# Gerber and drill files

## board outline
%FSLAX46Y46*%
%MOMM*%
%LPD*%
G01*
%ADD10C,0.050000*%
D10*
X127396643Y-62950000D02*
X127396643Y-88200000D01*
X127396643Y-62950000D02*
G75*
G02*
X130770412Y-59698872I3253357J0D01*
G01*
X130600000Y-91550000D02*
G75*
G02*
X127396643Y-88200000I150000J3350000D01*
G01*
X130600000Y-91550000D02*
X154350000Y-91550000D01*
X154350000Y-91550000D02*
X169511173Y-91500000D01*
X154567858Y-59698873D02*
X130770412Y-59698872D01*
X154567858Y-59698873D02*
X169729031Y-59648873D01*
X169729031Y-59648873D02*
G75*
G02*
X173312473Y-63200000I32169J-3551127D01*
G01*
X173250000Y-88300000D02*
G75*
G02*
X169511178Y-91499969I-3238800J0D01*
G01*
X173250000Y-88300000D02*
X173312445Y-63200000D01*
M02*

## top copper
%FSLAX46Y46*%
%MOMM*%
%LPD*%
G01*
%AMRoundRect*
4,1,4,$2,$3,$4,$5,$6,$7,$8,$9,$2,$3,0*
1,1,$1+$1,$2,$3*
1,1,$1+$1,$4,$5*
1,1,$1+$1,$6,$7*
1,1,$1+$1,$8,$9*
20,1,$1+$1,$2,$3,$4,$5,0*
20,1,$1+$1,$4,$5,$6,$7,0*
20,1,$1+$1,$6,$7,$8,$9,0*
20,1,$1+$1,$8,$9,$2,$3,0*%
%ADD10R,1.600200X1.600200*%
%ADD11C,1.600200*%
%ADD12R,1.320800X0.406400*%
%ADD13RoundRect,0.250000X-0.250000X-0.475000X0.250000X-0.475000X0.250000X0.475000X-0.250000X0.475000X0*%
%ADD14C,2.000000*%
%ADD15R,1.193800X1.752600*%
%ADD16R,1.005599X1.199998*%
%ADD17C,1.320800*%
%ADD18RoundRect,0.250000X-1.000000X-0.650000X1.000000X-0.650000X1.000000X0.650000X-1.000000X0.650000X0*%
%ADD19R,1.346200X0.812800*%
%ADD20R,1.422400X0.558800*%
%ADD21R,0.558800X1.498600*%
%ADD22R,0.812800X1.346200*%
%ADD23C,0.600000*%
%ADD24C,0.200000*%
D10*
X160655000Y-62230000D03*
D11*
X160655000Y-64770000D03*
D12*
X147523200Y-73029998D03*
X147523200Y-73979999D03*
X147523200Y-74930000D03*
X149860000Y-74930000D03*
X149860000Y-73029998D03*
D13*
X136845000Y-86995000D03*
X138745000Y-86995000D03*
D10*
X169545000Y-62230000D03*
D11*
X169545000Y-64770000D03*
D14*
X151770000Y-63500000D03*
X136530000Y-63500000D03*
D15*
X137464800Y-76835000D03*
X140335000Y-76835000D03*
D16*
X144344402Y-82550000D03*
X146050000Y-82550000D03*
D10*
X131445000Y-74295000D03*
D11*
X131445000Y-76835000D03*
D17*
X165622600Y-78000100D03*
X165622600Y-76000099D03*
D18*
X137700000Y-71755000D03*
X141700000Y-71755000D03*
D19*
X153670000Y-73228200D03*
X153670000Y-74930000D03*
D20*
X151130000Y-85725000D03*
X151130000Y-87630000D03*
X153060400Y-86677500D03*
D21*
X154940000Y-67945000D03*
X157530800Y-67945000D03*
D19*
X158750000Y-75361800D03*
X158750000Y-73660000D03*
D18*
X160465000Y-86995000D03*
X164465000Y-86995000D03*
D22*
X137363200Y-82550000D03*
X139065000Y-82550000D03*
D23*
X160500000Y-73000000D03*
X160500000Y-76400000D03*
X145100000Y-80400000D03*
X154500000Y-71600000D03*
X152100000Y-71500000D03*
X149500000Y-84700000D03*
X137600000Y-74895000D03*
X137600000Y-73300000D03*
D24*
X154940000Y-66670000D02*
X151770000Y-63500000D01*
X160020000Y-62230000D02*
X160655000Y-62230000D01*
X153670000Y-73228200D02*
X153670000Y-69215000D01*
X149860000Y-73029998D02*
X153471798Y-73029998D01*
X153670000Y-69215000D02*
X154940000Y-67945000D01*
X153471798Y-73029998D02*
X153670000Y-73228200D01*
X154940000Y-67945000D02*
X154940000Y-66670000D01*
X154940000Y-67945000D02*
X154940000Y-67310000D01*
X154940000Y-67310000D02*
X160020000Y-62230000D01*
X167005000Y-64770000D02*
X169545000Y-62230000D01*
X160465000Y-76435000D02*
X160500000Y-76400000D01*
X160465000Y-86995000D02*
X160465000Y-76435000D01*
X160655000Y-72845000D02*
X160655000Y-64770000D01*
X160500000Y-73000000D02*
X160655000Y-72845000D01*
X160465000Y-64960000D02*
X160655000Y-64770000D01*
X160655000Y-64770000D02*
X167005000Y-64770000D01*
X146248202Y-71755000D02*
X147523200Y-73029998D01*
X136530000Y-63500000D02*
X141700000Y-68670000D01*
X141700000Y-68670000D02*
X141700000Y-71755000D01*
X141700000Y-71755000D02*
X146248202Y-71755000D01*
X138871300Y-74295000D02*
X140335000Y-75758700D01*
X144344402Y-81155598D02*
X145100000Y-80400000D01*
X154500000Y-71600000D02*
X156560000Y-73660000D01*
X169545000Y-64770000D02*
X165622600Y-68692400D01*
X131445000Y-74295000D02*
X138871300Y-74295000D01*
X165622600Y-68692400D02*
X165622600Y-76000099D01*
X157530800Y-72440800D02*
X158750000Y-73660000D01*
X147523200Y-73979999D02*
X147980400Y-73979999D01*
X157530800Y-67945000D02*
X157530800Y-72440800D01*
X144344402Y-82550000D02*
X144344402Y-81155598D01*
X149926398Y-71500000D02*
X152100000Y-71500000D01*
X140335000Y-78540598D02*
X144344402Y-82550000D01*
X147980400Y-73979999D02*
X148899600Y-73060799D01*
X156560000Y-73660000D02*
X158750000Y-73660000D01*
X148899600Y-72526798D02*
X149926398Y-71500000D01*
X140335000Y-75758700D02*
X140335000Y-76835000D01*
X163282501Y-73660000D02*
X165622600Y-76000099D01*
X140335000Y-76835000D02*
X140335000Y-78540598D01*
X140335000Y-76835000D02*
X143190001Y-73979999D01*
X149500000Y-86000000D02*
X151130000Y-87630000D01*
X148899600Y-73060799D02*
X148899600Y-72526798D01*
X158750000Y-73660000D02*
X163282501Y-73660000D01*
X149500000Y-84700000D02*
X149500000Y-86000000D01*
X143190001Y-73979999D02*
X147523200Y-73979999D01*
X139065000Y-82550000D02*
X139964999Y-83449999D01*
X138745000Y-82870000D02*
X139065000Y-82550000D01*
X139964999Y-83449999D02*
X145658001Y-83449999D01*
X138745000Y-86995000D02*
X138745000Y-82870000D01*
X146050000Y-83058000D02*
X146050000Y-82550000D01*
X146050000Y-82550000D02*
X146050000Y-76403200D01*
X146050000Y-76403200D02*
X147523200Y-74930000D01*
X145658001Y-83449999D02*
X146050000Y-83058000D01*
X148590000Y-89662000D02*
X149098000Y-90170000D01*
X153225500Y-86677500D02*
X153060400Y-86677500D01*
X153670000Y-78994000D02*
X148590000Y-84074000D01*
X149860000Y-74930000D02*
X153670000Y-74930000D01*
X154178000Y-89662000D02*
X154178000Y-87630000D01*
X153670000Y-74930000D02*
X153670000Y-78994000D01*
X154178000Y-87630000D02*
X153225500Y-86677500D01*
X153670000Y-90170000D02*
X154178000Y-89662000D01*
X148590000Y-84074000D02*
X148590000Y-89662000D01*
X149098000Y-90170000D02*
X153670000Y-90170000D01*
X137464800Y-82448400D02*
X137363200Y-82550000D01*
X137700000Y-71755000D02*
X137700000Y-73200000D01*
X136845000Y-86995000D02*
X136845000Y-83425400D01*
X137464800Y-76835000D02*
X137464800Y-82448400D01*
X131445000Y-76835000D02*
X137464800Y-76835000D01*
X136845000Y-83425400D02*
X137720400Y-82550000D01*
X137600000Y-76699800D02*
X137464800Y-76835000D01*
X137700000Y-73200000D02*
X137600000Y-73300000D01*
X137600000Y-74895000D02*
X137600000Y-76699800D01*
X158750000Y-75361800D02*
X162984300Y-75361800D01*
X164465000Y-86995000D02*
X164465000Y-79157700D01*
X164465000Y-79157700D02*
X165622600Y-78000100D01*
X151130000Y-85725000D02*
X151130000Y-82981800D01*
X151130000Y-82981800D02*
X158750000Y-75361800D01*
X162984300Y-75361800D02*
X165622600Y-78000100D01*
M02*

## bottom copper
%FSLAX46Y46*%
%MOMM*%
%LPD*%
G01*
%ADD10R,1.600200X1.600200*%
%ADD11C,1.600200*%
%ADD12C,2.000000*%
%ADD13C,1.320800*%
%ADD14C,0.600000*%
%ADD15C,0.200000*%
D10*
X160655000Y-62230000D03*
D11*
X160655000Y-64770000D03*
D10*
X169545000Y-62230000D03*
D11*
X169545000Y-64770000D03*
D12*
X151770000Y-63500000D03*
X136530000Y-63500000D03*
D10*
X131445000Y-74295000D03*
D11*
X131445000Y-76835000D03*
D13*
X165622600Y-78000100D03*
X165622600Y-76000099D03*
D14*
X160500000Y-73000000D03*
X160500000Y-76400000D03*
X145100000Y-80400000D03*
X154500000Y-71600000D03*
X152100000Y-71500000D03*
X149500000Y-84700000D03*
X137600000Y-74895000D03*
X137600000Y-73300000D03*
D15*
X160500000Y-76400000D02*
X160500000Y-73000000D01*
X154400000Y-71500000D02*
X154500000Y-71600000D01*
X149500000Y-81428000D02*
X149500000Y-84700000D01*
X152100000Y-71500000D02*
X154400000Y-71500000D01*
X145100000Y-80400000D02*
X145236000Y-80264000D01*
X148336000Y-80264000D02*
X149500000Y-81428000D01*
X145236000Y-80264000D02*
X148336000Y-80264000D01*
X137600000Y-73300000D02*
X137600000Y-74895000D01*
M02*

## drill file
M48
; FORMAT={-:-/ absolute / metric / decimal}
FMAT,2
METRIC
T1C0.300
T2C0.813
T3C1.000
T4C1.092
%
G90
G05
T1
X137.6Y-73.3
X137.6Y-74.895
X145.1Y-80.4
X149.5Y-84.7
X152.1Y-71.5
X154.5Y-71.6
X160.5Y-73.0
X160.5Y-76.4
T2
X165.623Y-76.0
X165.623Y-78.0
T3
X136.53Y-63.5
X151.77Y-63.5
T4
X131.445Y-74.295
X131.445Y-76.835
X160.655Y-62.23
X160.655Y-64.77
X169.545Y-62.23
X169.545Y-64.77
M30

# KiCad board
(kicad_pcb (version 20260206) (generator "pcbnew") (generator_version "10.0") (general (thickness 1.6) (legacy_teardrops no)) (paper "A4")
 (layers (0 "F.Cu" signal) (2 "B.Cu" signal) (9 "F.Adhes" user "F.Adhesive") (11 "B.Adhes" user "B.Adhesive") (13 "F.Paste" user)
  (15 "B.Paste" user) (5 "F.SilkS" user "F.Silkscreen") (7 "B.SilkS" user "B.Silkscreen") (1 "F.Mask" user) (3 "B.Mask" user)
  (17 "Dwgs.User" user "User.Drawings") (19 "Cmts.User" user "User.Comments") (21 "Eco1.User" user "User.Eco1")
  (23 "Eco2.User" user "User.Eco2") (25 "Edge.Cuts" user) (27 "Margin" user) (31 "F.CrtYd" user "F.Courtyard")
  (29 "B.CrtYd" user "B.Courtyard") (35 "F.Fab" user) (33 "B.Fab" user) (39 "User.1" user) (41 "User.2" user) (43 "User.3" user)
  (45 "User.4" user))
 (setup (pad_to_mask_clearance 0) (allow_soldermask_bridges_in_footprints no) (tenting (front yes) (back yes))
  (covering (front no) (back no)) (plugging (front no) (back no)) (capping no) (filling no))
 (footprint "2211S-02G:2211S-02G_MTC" (layer "F.Cu") (at 160.655 62.23 90)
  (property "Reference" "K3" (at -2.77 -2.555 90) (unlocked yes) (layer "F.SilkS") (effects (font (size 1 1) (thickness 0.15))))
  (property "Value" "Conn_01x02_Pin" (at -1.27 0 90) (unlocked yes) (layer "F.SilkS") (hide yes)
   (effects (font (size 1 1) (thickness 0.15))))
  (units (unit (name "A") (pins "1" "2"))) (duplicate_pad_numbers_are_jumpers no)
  (pad "1" thru_hole rect (at 0 0 90) (size 1.6002 1.6002) (drill 1.0922) (layers "*.Cu" "*.Mask") (remove_unused_layers no) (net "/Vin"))
  (pad "2" thru_hole circle (at -2.54 0 90) (size 1.6002 1.6002) (drill 1.0922) (layers "*.Cu" "*.Mask") (remove_unused_layers no)
   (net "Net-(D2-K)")))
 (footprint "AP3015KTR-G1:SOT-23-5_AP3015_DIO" (layer "F.Cu") (at 148.6916 73.979999)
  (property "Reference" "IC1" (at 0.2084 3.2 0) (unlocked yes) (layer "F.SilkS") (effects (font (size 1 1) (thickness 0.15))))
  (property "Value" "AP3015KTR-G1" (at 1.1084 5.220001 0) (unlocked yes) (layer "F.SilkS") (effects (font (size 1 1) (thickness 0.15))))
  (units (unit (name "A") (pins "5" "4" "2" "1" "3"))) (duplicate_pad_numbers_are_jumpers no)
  (pad "1" smd rect (at -1.1684 -0.950001) (size 1.3208 0.4064) (layers "F.Cu" "F.Mask" "F.Paste") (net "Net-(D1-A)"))
  (pad "2" smd rect (at -1.1684 0) (size 1.3208 0.4064) (layers "F.Cu" "F.Mask" "F.Paste") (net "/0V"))
  (pad "3" smd rect (at -1.1684 0.950001) (size 1.3208 0.4064) (layers "F.Cu" "F.Mask" "F.Paste") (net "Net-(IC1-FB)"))
  (pad "4" smd rect (at 1.1684 0.950001) (size 1.3208 0.4064) (layers "F.Cu" "F.Mask" "F.Paste") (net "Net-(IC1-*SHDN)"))
  (pad "5" smd rect (at 1.1684 -0.950001) (size 1.3208 0.4064) (layers "F.Cu" "F.Mask" "F.Paste") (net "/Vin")))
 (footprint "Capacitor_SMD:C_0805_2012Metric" (layer "F.Cu") (at 137.795 86.995)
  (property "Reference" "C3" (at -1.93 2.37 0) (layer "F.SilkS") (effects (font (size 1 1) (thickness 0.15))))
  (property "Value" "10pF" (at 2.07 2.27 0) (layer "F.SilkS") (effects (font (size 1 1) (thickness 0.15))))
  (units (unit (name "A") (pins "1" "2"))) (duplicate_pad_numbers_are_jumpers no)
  (pad "1" smd roundrect (at -0.95 0) (size 1 1.45) (layers "F.Cu" "F.Mask" "F.Paste") (roundrect_rratio 0.25) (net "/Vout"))
  (pad "2" smd roundrect (at 0.95 0) (size 1 1.45) (layers "F.Cu" "F.Mask" "F.Paste") (roundrect_rratio 0.25) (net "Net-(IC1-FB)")))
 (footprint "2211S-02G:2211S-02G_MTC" (layer "F.Cu") (at 169.545 62.23 90)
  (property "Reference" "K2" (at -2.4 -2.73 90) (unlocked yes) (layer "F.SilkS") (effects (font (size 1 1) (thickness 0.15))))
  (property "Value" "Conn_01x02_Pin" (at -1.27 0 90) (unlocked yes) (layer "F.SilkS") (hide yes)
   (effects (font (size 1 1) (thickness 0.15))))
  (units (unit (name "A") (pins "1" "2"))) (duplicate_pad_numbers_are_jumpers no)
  (pad "1" thru_hole rect (at 0 0 90) (size 1.6002 1.6002) (drill 1.0922) (layers "*.Cu" "*.Mask") (remove_unused_layers no)
   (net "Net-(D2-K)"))
  (pad "2" thru_hole circle (at -2.54 0 90) (size 1.6002 1.6002) (drill 1.0922) (layers "*.Cu" "*.Mask") (remove_unused_layers no)
   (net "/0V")))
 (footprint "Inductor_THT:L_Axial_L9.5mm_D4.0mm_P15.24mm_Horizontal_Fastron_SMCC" (layer "F.Cu") (at 151.77 63.5 180)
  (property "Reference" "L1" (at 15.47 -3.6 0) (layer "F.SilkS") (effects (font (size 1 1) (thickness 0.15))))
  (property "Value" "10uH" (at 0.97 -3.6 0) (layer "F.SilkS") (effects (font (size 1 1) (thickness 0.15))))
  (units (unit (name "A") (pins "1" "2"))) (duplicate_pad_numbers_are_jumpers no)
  (pad "1" thru_hole circle (at 0 0 180) (size 2 2) (drill 1) (layers "*.Cu" "*.Mask") (remove_unused_layers no) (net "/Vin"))
  (pad "2" thru_hole circle (at 15.24 0 180) (size 2 2) (drill 1) (layers "*.Cu" "*.Mask") (remove_unused_layers no) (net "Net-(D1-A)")))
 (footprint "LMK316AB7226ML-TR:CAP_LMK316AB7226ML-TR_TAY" (layer "F.Cu") (at 138.8999 76.835)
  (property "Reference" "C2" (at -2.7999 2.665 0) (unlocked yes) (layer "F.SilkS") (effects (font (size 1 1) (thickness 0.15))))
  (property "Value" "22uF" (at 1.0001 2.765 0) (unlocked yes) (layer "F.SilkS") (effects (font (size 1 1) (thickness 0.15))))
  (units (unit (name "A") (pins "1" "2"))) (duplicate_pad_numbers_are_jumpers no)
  (pad "1" smd rect (at -1.4351 0) (size 1.1938 1.7526) (layers "F.Cu" "F.Mask" "F.Paste") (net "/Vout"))
  (pad "2" smd rect (at 1.4351 0) (size 1.1938 1.7526) (layers "F.Cu" "F.Mask" "F.Paste") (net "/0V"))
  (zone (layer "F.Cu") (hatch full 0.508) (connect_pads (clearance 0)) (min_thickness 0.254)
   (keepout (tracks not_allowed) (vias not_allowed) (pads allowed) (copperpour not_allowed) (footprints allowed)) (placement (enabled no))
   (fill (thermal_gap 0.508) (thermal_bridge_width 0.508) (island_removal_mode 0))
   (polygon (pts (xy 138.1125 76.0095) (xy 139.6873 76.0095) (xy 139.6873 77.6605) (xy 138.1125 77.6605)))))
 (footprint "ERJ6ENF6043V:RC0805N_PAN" (layer "F.Cu") (at 145.197201 82.55)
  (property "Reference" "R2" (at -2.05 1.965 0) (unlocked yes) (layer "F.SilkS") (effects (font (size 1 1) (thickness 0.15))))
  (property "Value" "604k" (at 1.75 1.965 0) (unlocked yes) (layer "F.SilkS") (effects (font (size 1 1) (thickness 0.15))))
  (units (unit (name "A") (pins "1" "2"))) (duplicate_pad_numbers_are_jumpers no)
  (pad "1" smd rect (at -0.852799 0) (size 1.005599 1.199998) (layers "F.Cu" "F.Mask" "F.Paste") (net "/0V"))
  (pad "2" smd rect (at 0.852799 0) (size 1.005599 1.199998) (layers "F.Cu" "F.Mask" "F.Paste") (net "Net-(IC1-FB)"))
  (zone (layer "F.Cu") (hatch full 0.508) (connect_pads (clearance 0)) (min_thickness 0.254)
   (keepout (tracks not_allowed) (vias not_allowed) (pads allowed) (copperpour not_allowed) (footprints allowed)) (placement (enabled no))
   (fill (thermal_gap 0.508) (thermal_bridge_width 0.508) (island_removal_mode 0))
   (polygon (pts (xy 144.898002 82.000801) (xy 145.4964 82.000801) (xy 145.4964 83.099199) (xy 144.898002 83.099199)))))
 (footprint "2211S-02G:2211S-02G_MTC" (layer "F.Cu") (at 131.445 74.295 90)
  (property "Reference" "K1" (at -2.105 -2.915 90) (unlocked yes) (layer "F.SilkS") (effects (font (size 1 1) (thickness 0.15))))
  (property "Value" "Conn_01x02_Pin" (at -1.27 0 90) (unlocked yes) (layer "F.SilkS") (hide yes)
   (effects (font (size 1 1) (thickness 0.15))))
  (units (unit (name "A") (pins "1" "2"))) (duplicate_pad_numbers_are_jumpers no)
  (pad "1" thru_hole rect (at 0 0 90) (size 1.6002 1.6002) (drill 1.0922) (layers "*.Cu" "*.Mask") (remove_unused_layers no) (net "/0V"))
  (pad "2" thru_hole circle (at -2.54 0 90) (size 1.6002 1.6002) (drill 1.0922) (layers "*.Cu" "*.Mask") (remove_unused_layers no)
   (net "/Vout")))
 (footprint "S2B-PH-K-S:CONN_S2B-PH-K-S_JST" (layer "F.Cu") (at 165.6226 78.0001 90)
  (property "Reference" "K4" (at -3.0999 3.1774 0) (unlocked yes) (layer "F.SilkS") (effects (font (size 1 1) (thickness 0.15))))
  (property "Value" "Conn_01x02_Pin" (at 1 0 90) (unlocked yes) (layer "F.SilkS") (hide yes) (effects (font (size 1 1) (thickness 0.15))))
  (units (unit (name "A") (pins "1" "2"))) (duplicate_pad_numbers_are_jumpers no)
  (pad "1" thru_hole circle (at 0 0 90) (size 1.3208 1.3208) (drill 0.8128) (layers "*.Cu" "*.Mask") (remove_unused_layers no) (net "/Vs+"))
  (pad "2" thru_hole circle (at 2.000001 0 90) (size 1.3208 1.3208) (drill 0.8128) (layers "*.Cu" "*.Mask") (remove_unused_layers no)
   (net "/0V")))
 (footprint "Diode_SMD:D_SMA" (layer "F.Cu") (at 139.7 71.755)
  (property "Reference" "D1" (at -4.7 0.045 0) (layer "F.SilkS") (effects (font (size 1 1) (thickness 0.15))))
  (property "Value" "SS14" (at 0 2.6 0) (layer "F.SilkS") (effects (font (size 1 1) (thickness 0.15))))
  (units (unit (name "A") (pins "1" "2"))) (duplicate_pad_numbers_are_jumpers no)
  (pad "1" smd roundrect (at -2 0) (size 2.5 1.8) (layers "F.Cu" "F.Mask" "F.Paste") (roundrect_rratio 0.1388888889) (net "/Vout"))
  (pad "2" smd roundrect (at 2 0) (size 2.5 1.8) (layers "F.Cu" "F.Mask" "F.Paste") (roundrect_rratio 0.1388888889) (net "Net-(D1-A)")))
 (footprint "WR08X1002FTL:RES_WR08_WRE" (layer "F.Cu") (at 153.67 74.0791 -90)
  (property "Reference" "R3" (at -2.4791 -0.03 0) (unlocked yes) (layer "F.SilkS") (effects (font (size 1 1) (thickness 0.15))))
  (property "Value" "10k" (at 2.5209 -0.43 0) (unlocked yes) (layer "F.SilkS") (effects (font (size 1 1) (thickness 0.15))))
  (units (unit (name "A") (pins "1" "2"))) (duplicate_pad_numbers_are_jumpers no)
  (pad "1" smd rect (at -0.8509 0 270) (size 0.8128 1.3462) (layers "F.Cu" "F.Mask" "F.Paste") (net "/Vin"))
  (pad "2" smd rect (at 0.8509 0 270) (size 0.8128 1.3462) (layers "F.Cu" "F.Mask" "F.Paste") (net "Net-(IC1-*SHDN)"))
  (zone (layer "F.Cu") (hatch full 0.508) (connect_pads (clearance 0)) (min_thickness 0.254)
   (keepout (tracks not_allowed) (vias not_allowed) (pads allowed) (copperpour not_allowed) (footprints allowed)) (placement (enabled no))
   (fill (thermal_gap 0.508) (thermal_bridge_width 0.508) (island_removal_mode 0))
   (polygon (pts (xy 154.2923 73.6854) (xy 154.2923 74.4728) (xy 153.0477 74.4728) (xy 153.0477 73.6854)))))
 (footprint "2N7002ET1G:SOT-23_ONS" (layer "F.Cu") (at 152.0952 86.6775 -90)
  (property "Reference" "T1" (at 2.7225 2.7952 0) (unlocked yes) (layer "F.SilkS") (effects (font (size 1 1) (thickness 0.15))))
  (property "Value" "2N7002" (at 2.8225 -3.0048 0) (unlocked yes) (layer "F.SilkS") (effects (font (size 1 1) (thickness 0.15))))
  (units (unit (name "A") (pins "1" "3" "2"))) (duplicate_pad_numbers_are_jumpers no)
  (pad "1" smd rect (at -0.9525 0.9652 270) (size 0.5588 1.4224) (layers "F.Cu" "F.Mask" "F.Paste") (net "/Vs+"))
  (pad "2" smd rect (at 0.9525 0.9652 270) (size 0.5588 1.4224) (layers "F.Cu" "F.Mask" "F.Paste") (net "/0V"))
  (pad "3" smd rect (at 0 -0.9652 270) (size 0.5588 1.4224) (layers "F.Cu" "F.Mask" "F.Paste") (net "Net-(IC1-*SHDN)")))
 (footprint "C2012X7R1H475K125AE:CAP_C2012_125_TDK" (layer "F.Cu") (at 156.2354 67.945)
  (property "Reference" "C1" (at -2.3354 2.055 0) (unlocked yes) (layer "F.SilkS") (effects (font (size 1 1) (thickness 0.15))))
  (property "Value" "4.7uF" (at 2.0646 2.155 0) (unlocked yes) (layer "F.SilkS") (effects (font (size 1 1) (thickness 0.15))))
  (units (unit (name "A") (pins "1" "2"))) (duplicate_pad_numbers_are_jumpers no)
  (pad "1" smd rect (at -1.2954 0) (size 0.5588 1.4986) (layers "F.Cu" "F.Mask" "F.Paste") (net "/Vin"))
  (pad "2" smd rect (at 1.2954 0) (size 0.5588 1.4986) (layers "F.Cu" "F.Mask" "F.Paste") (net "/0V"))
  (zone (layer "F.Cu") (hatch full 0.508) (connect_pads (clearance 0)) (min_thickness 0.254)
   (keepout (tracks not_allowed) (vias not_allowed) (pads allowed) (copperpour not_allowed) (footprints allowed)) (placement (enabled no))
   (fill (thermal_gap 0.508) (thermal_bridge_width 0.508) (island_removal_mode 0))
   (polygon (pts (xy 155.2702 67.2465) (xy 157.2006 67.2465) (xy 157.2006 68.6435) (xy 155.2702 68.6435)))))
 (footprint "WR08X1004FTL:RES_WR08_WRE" (layer "F.Cu") (at 158.75 74.5109 90)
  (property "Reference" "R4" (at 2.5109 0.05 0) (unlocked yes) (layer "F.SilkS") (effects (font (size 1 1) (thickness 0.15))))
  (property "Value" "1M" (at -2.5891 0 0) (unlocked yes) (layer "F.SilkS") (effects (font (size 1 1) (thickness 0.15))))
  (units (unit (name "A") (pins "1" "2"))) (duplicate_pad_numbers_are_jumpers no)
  (pad "1" smd rect (at -0.8509 0 90) (size 0.8128 1.3462) (layers "F.Cu" "F.Mask" "F.Paste") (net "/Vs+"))
  (pad "2" smd rect (at 0.8509 0 90) (size 0.8128 1.3462) (layers "F.Cu" "F.Mask" "F.Paste") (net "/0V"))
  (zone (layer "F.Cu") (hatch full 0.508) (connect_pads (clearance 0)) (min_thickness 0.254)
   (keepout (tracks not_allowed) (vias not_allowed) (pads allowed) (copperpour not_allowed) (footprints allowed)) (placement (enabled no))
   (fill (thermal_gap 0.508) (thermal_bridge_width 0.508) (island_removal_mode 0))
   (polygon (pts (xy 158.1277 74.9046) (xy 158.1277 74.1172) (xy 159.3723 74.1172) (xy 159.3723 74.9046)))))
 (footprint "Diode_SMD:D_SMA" (layer "F.Cu") (at 162.465 86.995)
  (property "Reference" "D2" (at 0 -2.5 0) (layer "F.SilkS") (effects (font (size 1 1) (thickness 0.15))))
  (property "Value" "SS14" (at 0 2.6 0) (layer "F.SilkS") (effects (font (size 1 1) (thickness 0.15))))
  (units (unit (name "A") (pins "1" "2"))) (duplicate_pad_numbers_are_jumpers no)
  (pad "1" smd roundrect (at -2 0) (size 2.5 1.8) (layers "F.Cu" "F.Mask" "F.Paste") (roundrect_rratio 0.1388888889) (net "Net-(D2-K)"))
  (pad "2" smd roundrect (at 2 0) (size 2.5 1.8) (layers "F.Cu" "F.Mask" "F.Paste") (roundrect_rratio 0.1388888889) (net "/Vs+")))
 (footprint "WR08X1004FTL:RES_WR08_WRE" (layer "F.Cu") (at 138.2141 82.55)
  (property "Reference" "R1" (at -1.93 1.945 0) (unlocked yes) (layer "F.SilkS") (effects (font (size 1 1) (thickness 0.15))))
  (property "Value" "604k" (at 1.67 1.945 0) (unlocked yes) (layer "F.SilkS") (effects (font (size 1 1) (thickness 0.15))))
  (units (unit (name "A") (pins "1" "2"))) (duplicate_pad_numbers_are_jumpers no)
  (pad "1" smd rect (at -0.8509 0) (size 0.8128 1.3462) (layers "F.Cu" "F.Mask" "F.Paste") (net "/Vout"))
  (pad "2" smd rect (at 0.8509 0) (size 0.8128 1.3462) (layers "F.Cu" "F.Mask" "F.Paste") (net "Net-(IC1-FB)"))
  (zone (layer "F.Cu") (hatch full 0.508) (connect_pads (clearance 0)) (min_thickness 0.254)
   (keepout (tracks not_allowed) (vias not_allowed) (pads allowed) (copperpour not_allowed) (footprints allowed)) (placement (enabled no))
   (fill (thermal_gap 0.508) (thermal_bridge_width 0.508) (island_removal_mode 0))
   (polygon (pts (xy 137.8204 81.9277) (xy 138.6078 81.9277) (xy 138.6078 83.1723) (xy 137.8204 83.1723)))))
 (gr_line (start 127.396643 62.95) (end 127.396643 88.2) (stroke (width 0.05) (type default)) (layer "Edge.Cuts"))
 (gr_arc (start 127.396643 62.95) (mid 128.392503 60.607344) (end 130.770412 59.698872) (stroke (width 0.05) (type default))
  (layer "Edge.Cuts"))
 (gr_arc (start 130.6 91.55) (mid 128.326366 90.517541) (end 127.396643 88.2) (stroke (width 0.05) (type default)) (layer "Edge.Cuts"))
 (gr_line (start 130.6 91.55) (end 154.35 91.55) (stroke (width 0.05) (type default)) (layer "Edge.Cuts"))
 (gr_line (start 154.35 91.55) (end 169.511173 91.5) (stroke (width 0.05) (type default)) (layer "Edge.Cuts"))
 (gr_line (start 154.567858 59.698873) (end 130.770412 59.698872) (stroke (width 0.05) (type default)) (layer "Edge.Cuts"))
 (gr_line (start 154.567858 59.698873) (end 169.729031 59.648873) (stroke (width 0.05) (type default)) (layer "Edge.Cuts"))
 (gr_arc (start 169.729031 59.648873) (mid 172.260912 60.677533) (end 173.312445 63.2) (stroke (width 0.05) (type default))
  (layer "Edge.Cuts"))
 (gr_arc (start 173.25 88.3) (mid 172.117187 90.760631) (end 169.511173 91.5) (stroke (width 0.05) (type default)) (layer "Edge.Cuts"))
 (gr_line (start 173.25 88.3) (end 173.312445 63.2) (stroke (width 0.05) (type default)) (layer "Edge.Cuts"))
 (segment (start 154.94 66.67) (end 151.77 63.5) (width 0.2) (layer "F.Cu") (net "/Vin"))
 (segment (start 160.02 62.23) (end 160.655 62.23) (width 0.2) (layer "F.Cu") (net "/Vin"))
 (segment (start 153.67 73.2282) (end 153.67 69.215) (width 0.2) (layer "F.Cu") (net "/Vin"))
 (segment (start 149.86 73.029998) (end 153.471798 73.029998) (width 0.2) (layer "F.Cu") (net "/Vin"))
 (segment (start 153.67 69.215) (end 154.94 67.945) (width 0.2) (layer "F.Cu") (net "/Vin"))
 (segment (start 153.471798 73.029998) (end 153.67 73.2282) (width 0.2) (layer "F.Cu") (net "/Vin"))
 (segment (start 154.94 67.945) (end 154.94 66.67) (width 0.2) (layer "F.Cu") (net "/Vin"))
 (segment (start 154.94 67.945) (end 154.94 67.31) (width 0.2) (layer "F.Cu") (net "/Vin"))
 (segment (start 154.94 67.31) (end 160.02 62.23) (width 0.2) (layer "F.Cu") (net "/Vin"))
 (segment (start 167.005 64.77) (end 169.545 62.23) (width 0.2) (layer "F.Cu") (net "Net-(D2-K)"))
 (segment (start 160.465 76.435) (end 160.5 76.4) (width 0.2) (layer "F.Cu") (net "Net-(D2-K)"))
 (segment (start 160.465 86.995) (end 160.465 76.435) (width 0.2) (layer "F.Cu") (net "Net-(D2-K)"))
 (segment (start 160.655 72.845) (end 160.655 64.77) (width 0.2) (layer "F.Cu") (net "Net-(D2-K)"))
 (segment (start 160.5 73) (end 160.655 72.845) (width 0.2) (layer "F.Cu") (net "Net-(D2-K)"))
 (segment (start 160.465 64.96) (end 160.655 64.77) (width 0.2) (layer "F.Cu") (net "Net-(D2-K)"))
 (segment (start 160.655 64.77) (end 167.005 64.77) (width 0.2) (layer "F.Cu") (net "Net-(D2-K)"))
 (via (at 160.5 73) (size 0.6) (drill 0.3) (layers "F.Cu" "B.Cu") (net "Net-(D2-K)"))
 (via (at 160.5 76.4) (size 0.6) (drill 0.3) (layers "F.Cu" "B.Cu") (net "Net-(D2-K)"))
 (segment (start 160.5 76.4) (end 160.5 73) (width 0.2) (layer "B.Cu") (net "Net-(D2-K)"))
 (segment (start 146.248202 71.755) (end 147.5232 73.029998) (width 0.2) (layer "F.Cu") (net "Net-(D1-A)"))
 (segment (start 136.53 63.5) (end 141.7 68.67) (width 0.2) (layer "F.Cu") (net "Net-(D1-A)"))
 (segment (start 141.7 68.67) (end 141.7 71.755) (width 0.2) (layer "F.Cu") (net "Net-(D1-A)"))
 (segment (start 141.7 71.755) (end 146.248202 71.755) (width 0.2) (layer "F.Cu") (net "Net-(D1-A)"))
 (segment (start 138.8713 74.295) (end 140.335 75.7587) (width 0.2) (layer "F.Cu") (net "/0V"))
 (segment (start 144.344402 81.155598) (end 145.1 80.4) (width 0.2) (layer "F.Cu") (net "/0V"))
 (segment (start 154.5 71.6) (end 156.56 73.66) (width 0.2) (layer "F.Cu") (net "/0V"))
 (segment (start 169.545 64.77) (end 165.6226 68.6924) (width 0.2) (layer "F.Cu") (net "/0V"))
 (segment (start 131.445 74.295) (end 138.8713 74.295) (width 0.2) (layer "F.Cu") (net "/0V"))
 (segment (start 165.6226 68.6924) (end 165.6226 76.000099) (width 0.2) (layer "F.Cu") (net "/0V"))
 (segment (start 157.5308 72.4408) (end 158.75 73.66) (width 0.2) (layer "F.Cu") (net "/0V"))
 (segment (start 147.5232 73.979999) (end 147.9804 73.979999) (width 0.2) (layer "F.Cu") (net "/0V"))
 (segment (start 157.5308 67.945) (end 157.5308 72.4408) (width 0.2) (layer "F.Cu") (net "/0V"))
 (segment (start 144.344402 82.55) (end 144.344402 81.155598) (width 0.2) (layer "F.Cu") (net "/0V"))
 (segment (start 149.926398 71.5) (end 152.1 71.5) (width 0.2) (layer "F.Cu") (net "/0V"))
 (segment (start 140.335 78.540598) (end 144.344402 82.55) (width 0.2) (layer "F.Cu") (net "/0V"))
 (segment (start 147.9804 73.979999) (end 148.8996 73.060799) (width 0.2) (layer "F.Cu") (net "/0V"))
 (segment (start 156.56 73.66) (end 158.75 73.66) (width 0.2) (layer "F.Cu") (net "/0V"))
 (segment (start 148.8996 72.526798) (end 149.926398 71.5) (width 0.2) (layer "F.Cu") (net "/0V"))
 (segment (start 140.335 75.7587) (end 140.335 76.835) (width 0.2) (layer "F.Cu") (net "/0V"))
 (segment (start 163.282501 73.66) (end 165.6226 76.000099) (width 0.2) (layer "F.Cu") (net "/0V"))
 (segment (start 140.335 76.835) (end 140.335 78.540598) (width 0.2) (layer "F.Cu") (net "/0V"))
 (segment (start 140.335 76.835) (end 143.190001 73.979999) (width 0.2) (layer "F.Cu") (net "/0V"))
 (segment (start 149.5 86) (end 151.13 87.63) (width 0.2) (layer "F.Cu") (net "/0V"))
 (segment (start 148.8996 73.060799) (end 148.8996 72.526798) (width 0.2) (layer "F.Cu") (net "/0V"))
 (segment (start 158.75 73.66) (end 163.282501 73.66) (width 0.2) (layer "F.Cu") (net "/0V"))
 (segment (start 149.5 84.7) (end 149.5 86) (width 0.2) (layer "F.Cu") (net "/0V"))
 (segment (start 143.190001 73.979999) (end 147.5232 73.979999) (width 0.2) (layer "F.Cu") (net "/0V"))
 (via (at 145.1 80.4) (size 0.6) (drill 0.3) (layers "F.Cu" "B.Cu") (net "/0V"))
 (via (at 154.5 71.6) (size 0.6) (drill 0.3) (layers "F.Cu" "B.Cu") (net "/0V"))
 (via (at 152.1 71.5) (size 0.6) (drill 0.3) (layers "F.Cu" "B.Cu") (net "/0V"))
 (via (at 149.5 84.7) (size 0.6) (drill 0.3) (layers "F.Cu" "B.Cu") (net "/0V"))
 (segment (start 154.4 71.5) (end 154.5 71.6) (width 0.2) (layer "B.Cu") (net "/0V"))
 (segment (start 149.5 81.428) (end 149.5 84.7) (width 0.2) (layer "B.Cu") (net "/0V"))
 (segment (start 152.1 71.5) (end 154.4 71.5) (width 0.2) (layer "B.Cu") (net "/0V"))
 (segment (start 145.1 80.4) (end 145.236 80.264) (width 0.2) (layer "B.Cu") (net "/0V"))
 (segment (start 148.336 80.264) (end 149.5 81.428) (width 0.2) (layer "B.Cu") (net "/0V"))
 (segment (start 145.236 80.264) (end 148.336 80.264) (width 0.2) (layer "B.Cu") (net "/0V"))
 (segment (start 139.065 82.55) (end 139.964999 83.449999) (width 0.2) (layer "F.Cu") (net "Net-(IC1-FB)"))
 (segment (start 138.745 82.87) (end 139.065 82.55) (width 0.2) (layer "F.Cu") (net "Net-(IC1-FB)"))
 (segment (start 139.964999 83.449999) (end 145.658001 83.449999) (width 0.2) (layer "F.Cu") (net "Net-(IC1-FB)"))
 (segment (start 138.745 86.995) (end 138.745 82.87) (width 0.2) (layer "F.Cu") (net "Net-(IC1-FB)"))
 (segment (start 146.05 83.058) (end 146.05 82.55) (width 0.2) (layer "F.Cu") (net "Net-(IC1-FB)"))
 (segment (start 146.05 82.55) (end 146.05 76.4032) (width 0.2) (layer "F.Cu") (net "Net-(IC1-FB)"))
 (segment (start 146.05 76.4032) (end 147.5232 74.93) (width 0.2) (layer "F.Cu") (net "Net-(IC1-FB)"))
 (segment (start 145.658001 83.449999) (end 146.05 83.058) (width 0.2) (layer "F.Cu") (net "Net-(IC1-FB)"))
 (segment (start 148.59 89.662) (end 149.098 90.17) (width 0.2) (layer "F.Cu") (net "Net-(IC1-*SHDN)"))
 (segment (start 153.2255 86.6775) (end 153.0604 86.6775) (width 0.2) (layer "F.Cu") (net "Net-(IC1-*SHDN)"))
 (segment (start 153.67 78.994) (end 148.59 84.074) (width 0.2) (layer "F.Cu") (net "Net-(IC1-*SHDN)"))
 (segment (start 149.86 74.93) (end 153.67 74.93) (width 0.2) (layer "F.Cu") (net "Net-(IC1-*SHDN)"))
 (segment (start 154.178 89.662) (end 154.178 87.63) (width 0.2) (layer "F.Cu") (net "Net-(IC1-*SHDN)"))
 (segment (start 153.67 74.93) (end 153.67 78.994) (width 0.2) (layer "F.Cu") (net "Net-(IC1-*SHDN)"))
 (segment (start 154.178 87.63) (end 153.2255 86.6775) (width 0.2) (layer "F.Cu") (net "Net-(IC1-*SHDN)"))
 (segment (start 153.67 90.17) (end 154.178 89.662) (width 0.2) (layer "F.Cu") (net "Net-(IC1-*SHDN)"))
 (segment (start 148.59 84.074) (end 148.59 89.662) (width 0.2) (layer "F.Cu") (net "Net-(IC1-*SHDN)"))
 (segment (start 149.098 90.17) (end 153.67 90.17) (width 0.2) (layer "F.Cu") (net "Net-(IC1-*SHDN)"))
 (segment (start 137.4648 82.4484) (end 137.3632 82.55) (width 0.2) (layer "F.Cu") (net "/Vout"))
 (segment (start 137.7 71.755) (end 137.7 73.2) (width 0.2) (layer "F.Cu") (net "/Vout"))
 (segment (start 136.845 86.995) (end 136.845 83.4254) (width 0.2) (layer "F.Cu") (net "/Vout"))
 (segment (start 137.4648 76.835) (end 137.4648 82.4484) (width 0.2) (layer "F.Cu") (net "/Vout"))
 (segment (start 131.445 76.835) (end 137.4648 76.835) (width 0.2) (layer "F.Cu") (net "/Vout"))
 (segment (start 136.845 83.4254) (end 137.7204 82.55) (width 0.2) (layer "F.Cu") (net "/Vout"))
 (segment (start 137.6 76.6998) (end 137.4648 76.835) (width 0.2) (layer "F.Cu") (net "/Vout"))
 (segment (start 137.7 73.2) (end 137.6 73.3) (width 0.2) (layer "F.Cu") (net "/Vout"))
 (segment (start 137.6 74.895) (end 137.6 76.6998) (width 0.2) (layer "F.Cu") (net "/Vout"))
 (via (at 137.6 74.895) (size 0.6) (drill 0.3) (layers "F.Cu" "B.Cu") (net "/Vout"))
 (via (at 137.6 73.3) (size 0.6) (drill 0.3) (layers "F.Cu" "B.Cu") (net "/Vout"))
 (segment (start 137.6 73.3) (end 137.6 74.895) (width 0.2) (layer "B.Cu") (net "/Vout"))
 (segment (start 158.75 75.3618) (end 162.9843 75.3618) (width 0.2) (layer "F.Cu") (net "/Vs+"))
 (segment (start 164.465 86.995) (end 164.465 79.1577) (width 0.2) (layer "F.Cu") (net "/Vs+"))
 (segment (start 164.465 79.1577) (end 165.6226 78.0001) (width 0.2) (layer "F.Cu") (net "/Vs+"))
 (segment (start 151.13 85.725) (end 151.13 82.9818) (width 0.2) (layer "F.Cu") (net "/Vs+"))
 (segment (start 151.13 82.9818) (end 158.75 75.3618) (width 0.2) (layer "F.Cu") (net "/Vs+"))
 (segment (start 162.9843 75.3618) (end 165.6226 78.0001) (width 0.2) (layer "F.Cu") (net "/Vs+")))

